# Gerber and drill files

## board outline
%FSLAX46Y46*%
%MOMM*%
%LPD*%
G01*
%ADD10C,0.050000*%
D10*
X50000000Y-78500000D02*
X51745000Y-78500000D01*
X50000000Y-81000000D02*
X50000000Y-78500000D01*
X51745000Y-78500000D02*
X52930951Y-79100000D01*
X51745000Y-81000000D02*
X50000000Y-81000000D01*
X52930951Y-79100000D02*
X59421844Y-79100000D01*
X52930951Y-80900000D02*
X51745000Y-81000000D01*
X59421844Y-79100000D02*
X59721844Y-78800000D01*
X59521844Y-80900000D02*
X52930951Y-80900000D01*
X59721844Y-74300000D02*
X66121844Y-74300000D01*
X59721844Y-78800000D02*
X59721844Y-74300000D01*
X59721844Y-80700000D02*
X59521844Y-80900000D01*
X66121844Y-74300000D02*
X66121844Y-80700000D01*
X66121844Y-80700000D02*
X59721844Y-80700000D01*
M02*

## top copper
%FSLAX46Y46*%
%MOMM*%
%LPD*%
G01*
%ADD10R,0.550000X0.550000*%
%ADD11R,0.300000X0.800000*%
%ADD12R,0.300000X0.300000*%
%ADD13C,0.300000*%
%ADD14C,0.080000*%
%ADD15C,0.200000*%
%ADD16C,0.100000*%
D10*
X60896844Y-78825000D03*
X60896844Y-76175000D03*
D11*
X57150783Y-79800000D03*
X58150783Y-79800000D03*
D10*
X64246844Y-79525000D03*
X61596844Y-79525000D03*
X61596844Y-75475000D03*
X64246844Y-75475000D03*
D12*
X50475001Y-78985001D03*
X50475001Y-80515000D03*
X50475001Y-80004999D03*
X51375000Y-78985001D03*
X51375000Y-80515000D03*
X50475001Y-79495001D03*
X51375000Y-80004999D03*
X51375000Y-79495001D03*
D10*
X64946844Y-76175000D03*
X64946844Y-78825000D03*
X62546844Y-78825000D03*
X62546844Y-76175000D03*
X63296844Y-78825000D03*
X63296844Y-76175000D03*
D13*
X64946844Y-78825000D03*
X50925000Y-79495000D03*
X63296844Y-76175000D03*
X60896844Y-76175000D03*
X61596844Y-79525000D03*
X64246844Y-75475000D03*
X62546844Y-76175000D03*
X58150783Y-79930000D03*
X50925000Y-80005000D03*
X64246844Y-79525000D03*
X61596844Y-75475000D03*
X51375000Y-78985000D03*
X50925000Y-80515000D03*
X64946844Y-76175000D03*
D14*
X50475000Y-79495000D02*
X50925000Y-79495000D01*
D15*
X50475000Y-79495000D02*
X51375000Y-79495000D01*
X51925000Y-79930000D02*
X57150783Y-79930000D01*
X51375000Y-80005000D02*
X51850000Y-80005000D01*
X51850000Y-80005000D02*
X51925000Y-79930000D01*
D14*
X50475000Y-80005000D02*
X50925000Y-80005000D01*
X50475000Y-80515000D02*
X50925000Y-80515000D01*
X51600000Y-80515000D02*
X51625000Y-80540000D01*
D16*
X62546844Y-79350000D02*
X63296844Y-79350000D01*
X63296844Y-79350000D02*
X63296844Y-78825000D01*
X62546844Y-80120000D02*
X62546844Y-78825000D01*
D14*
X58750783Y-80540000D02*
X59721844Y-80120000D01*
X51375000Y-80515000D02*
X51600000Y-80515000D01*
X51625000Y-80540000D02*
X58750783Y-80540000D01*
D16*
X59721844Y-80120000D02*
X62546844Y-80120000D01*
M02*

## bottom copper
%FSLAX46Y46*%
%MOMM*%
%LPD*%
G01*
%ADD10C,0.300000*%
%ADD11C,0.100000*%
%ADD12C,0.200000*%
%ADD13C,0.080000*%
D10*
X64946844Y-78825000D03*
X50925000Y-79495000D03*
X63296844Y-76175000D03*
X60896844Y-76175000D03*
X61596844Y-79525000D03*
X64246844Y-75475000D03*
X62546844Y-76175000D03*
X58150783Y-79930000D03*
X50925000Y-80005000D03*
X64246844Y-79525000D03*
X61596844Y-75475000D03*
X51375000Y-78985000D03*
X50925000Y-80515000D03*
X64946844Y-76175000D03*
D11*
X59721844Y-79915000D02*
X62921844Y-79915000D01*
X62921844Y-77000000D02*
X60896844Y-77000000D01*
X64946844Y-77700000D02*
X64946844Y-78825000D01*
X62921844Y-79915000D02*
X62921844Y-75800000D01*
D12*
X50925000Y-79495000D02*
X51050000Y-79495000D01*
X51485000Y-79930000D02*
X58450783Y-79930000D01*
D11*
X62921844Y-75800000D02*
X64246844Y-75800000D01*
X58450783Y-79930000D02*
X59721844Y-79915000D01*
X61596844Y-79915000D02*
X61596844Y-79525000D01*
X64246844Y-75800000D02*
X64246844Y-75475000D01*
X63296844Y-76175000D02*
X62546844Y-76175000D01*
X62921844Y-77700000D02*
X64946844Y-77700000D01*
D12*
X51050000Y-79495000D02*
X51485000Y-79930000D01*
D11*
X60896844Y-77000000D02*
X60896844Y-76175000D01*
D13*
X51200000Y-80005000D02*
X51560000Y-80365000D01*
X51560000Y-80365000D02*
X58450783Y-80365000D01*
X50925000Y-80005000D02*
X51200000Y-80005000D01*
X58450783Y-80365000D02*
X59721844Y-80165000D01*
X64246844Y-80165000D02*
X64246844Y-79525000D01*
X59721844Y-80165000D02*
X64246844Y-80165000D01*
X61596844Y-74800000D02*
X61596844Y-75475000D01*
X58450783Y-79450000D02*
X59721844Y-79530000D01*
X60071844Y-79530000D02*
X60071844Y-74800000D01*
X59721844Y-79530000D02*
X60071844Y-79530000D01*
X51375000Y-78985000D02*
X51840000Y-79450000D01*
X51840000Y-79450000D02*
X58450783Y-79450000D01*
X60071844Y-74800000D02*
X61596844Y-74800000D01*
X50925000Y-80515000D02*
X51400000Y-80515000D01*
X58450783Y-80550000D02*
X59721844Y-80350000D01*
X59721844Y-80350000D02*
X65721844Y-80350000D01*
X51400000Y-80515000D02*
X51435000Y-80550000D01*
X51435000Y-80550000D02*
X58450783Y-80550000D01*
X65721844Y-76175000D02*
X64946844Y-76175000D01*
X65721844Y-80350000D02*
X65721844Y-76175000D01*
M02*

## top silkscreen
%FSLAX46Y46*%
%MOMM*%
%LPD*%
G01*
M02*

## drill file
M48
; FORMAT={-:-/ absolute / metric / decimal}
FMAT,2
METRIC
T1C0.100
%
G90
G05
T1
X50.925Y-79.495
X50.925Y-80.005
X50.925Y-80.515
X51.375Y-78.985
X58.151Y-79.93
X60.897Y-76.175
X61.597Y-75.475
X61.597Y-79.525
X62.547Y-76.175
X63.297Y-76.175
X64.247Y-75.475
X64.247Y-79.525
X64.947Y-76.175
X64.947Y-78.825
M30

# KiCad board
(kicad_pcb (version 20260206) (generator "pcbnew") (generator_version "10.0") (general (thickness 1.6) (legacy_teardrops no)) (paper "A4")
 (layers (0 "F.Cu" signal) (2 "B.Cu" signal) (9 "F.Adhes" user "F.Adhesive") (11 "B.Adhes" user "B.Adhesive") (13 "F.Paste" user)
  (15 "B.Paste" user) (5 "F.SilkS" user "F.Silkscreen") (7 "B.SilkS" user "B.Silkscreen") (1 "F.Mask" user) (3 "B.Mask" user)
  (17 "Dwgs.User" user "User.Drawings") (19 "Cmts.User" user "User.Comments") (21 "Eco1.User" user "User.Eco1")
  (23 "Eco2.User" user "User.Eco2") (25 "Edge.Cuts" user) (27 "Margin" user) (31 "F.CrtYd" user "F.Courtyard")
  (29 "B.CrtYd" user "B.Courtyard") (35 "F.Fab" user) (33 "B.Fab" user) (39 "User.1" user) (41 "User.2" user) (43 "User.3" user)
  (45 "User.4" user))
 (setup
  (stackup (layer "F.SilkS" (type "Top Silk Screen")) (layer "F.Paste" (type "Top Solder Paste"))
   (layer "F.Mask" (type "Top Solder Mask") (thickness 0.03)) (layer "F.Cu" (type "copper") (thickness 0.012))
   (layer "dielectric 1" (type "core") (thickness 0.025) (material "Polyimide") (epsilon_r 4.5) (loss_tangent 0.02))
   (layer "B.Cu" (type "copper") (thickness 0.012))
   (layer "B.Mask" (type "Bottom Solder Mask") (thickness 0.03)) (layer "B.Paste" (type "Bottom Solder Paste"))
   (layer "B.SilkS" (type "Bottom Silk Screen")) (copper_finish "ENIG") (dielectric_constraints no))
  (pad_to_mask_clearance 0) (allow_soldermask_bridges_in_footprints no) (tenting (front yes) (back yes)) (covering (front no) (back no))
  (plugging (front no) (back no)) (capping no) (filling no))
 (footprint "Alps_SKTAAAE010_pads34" (layer "F.Cu") (at 60.521844 77.5 90)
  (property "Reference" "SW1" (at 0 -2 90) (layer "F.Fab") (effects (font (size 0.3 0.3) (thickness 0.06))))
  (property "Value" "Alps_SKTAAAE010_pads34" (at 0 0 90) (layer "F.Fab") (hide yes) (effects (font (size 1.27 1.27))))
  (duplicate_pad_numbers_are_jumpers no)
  (pad "3" smd rect (at -1.325 0.375 90) (size 0.55 0.55) (layers "F.Cu" "F.Mask") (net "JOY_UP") (solder_mask_margin 0.05)
   (thermal_bridge_angle 45))
  (pad "4" smd rect (at 1.325 0.375 90) (size 0.55 0.55) (layers "F.Cu" "F.Mask") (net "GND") (solder_mask_margin 0.05)
   (thermal_bridge_angle 45)))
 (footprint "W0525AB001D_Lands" (layer "F.Cu") (at 57.650783 79.93)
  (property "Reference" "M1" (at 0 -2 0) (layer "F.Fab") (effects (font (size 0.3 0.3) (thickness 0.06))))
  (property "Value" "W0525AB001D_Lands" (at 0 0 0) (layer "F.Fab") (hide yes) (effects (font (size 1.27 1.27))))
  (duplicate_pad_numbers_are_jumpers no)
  (pad "1" smd rect (at -0.5 -0.13) (size 0.3 0.8) (layers "F.Cu" "F.Mask") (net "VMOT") (solder_mask_margin 0.05) (thermal_bridge_angle 45))
  (pad "2" smd rect (at 0.5 -0.13) (size 0.3 0.8) (layers "F.Cu" "F.Mask") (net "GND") (solder_mask_margin 0.05) (thermal_bridge_angle 45)))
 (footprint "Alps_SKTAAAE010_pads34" (layer "F.Cu") (at 62.921844 79.9 180)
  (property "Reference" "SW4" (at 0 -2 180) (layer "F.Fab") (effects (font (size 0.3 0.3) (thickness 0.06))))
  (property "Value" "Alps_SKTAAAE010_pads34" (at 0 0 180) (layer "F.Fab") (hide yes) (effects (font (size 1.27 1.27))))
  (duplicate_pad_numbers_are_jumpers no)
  (pad "3" smd rect (at -1.325 0.375 180) (size 0.55 0.55) (layers "F.Cu" "F.Mask") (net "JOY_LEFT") (solder_mask_margin 0.05)
   (thermal_bridge_angle 45))
  (pad "4" smd rect (at 1.325 0.375 180) (size 0.55 0.55) (layers "F.Cu" "F.Mask") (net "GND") (solder_mask_margin 0.05)
   (thermal_bridge_angle 45)))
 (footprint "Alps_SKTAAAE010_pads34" (layer "F.Cu") (at 62.921844 75.1)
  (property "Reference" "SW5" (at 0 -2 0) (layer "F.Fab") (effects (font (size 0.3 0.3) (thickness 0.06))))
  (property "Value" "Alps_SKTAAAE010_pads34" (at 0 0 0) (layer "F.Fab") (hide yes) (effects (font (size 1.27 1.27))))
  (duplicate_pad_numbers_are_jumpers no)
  (pad "3" smd rect (at -1.325 0.375) (size 0.55 0.55) (layers "F.Cu" "F.Mask") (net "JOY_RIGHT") (solder_mask_margin 0.05)
   (thermal_bridge_angle 45))
  (pad "4" smd rect (at 1.325 0.375) (size 0.55 0.55) (layers "F.Cu" "F.Mask") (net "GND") (solder_mask_margin 0.05)
   (thermal_bridge_angle 45)))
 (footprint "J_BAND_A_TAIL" (layer "F.Cu") (at 50.9 79.75)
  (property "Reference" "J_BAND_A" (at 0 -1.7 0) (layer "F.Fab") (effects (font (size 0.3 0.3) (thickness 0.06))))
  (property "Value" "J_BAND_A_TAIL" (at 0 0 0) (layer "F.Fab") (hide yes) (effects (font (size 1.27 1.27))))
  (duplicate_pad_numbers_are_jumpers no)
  (pad "1" smd rect (at -0.424999 -0.764999) (size 0.3 0.3) (layers "F.Cu" "F.Mask") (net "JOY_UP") (solder_mask_margin 0.05)
   (thermal_bridge_angle 45))
  (pad "2" smd rect (at -0.424999 0.765) (size 0.3 0.3) (layers "F.Cu" "F.Mask") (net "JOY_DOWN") (solder_mask_margin 0.05)
   (thermal_bridge_angle 45))
  (pad "3" smd rect (at -0.424999 0.254999) (size 0.3 0.3) (layers "F.Cu" "F.Mask") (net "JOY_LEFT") (solder_mask_margin 0.05)
   (thermal_bridge_angle 45))
  (pad "4" smd rect (at 0.475 -0.764999) (size 0.3 0.3) (layers "F.Cu" "F.Mask") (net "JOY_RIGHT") (solder_mask_margin 0.05)
   (thermal_bridge_angle 45))
  (pad "5" smd rect (at 0.475 0.765) (size 0.3 0.3) (layers "F.Cu" "F.Mask") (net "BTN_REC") (solder_mask_margin 0.05)
   (thermal_bridge_angle 45))
  (pad "6" smd rect (at -0.424999 -0.254999) (size 0.3 0.3) (layers "F.Cu" "F.Mask") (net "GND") (solder_mask_margin 0.05)
   (thermal_bridge_angle 45))
  (pad "7" smd rect (at 0.475 0.254999) (size 0.3 0.3) (layers "F.Cu" "F.Mask") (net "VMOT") (solder_mask_margin 0.05)
   (thermal_bridge_angle 45))
  (pad "8" smd rect (at 0.475 -0.254999) (size 0.3 0.3) (layers "F.Cu" "F.Mask") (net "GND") (solder_mask_margin 0.05)
   (thermal_bridge_angle 45)))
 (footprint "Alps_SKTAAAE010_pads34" (layer "F.Cu") (at 65.321844 77.5 -90)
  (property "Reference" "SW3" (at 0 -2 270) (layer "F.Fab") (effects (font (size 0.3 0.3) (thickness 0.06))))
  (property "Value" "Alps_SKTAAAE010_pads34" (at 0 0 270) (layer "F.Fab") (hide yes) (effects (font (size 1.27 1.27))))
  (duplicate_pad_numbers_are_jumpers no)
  (pad "3" smd rect (at -1.325 0.375 270) (size 0.55 0.55) (layers "F.Cu" "F.Mask") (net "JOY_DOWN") (solder_mask_margin 0.05)
   (thermal_bridge_angle 45))
  (pad "4" smd rect (at 1.325 0.375 270) (size 0.55 0.55) (layers "F.Cu" "F.Mask") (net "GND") (solder_mask_margin 0.05)
   (thermal_bridge_angle 45)))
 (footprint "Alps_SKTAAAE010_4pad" (layer "F.Cu") (at 62.921844 77.5 90)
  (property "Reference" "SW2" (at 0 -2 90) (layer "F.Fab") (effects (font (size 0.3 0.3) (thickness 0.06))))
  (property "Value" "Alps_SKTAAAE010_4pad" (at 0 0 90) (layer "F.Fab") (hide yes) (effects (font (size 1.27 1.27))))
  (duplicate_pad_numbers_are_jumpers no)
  (pad "1" smd rect (at -1.325 -0.375 90) (size 0.55 0.55) (layers "F.Cu" "F.Mask") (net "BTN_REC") (solder_mask_margin 0.05)
   (thermal_bridge_angle 45))
  (pad "2" smd rect (at 1.325 -0.375 90) (size 0.55 0.55) (layers "F.Cu" "F.Mask") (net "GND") (solder_mask_margin 0.05)
   (thermal_bridge_angle 45))
  (pad "3" smd rect (at -1.325 0.375 90) (size 0.55 0.55) (layers "F.Cu" "F.Mask") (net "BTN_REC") (solder_mask_margin 0.05)
   (thermal_bridge_angle 45))
  (pad "4" smd rect (at 1.325 0.375 90) (size 0.55 0.55) (layers "F.Cu" "F.Mask") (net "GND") (solder_mask_margin 0.05)
   (thermal_bridge_angle 45)))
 (gr_line (start 50 78.5) (end 51.745 78.5) (stroke (width 0.05) (type default)) (layer "Edge.Cuts"))
 (gr_line (start 50 81) (end 50 78.5) (stroke (width 0.05) (type default)) (layer "Edge.Cuts"))
 (gr_line (start 51.745 78.5) (end 52.930951 79.1) (stroke (width 0.05) (type default)) (layer "Edge.Cuts"))
 (gr_line (start 51.745 81) (end 50 81) (stroke (width 0.05) (type default)) (layer "Edge.Cuts"))
 (gr_line (start 52.930951 79.1) (end 59.421844 79.1) (stroke (width 0.05) (type default)) (layer "Edge.Cuts"))
 (gr_line (start 52.930951 80.9) (end 51.745 81) (stroke (width 0.05) (type default)) (layer "Edge.Cuts"))
 (gr_line (start 59.421844 79.1) (end 59.721844 78.8) (stroke (width 0.05) (type default)) (layer "Edge.Cuts"))
 (gr_line (start 59.521844 80.9) (end 52.930951 80.9) (stroke (width 0.05) (type default)) (layer "Edge.Cuts"))
 (gr_line (start 59.721844 74.3) (end 66.121844 74.3) (stroke (width 0.05) (type default)) (layer "Edge.Cuts"))
 (gr_line (start 59.721844 78.8) (end 59.721844 74.3) (stroke (width 0.05) (type default)) (layer "Edge.Cuts"))
 (gr_line (start 59.721844 80.7) (end 59.521844 80.9) (stroke (width 0.05) (type default)) (layer "Edge.Cuts"))
 (gr_line (start 66.121844 74.3) (end 66.121844 80.7) (stroke (width 0.05) (type default)) (layer "Edge.Cuts"))
 (gr_line (start 66.121844 80.7) (end 59.721844 80.7) (stroke (width 0.05) (type default)) (layer "Edge.Cuts"))
 (segment (start 50.475 79.495) (end 50.925 79.495) (width 0.08) (layer "F.Cu") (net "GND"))
 (segment (start 50.475 79.495) (end 51.375 79.495) (width 0.2) (layer "F.Cu") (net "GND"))
 (via (at 64.946844 78.825) (size 0.3) (drill 0.1) (layers "F.Cu" "B.Cu") (tenting (front yes) (back yes)) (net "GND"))
 (via (at 50.925 79.495) (size 0.3) (drill 0.1) (layers "F.Cu" "B.Cu") (tenting (front yes) (back yes)) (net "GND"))
 (via (at 63.296844 76.175) (size 0.3) (drill 0.1) (layers "F.Cu" "B.Cu") (tenting (front yes) (back yes)) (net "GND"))
 (via (at 60.896844 76.175) (size 0.3) (drill 0.1) (layers "F.Cu" "B.Cu") (tenting (front yes) (back yes)) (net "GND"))
 (via (at 61.596844 79.525) (size 0.3) (drill 0.1) (layers "F.Cu" "B.Cu") (tenting (front yes) (back yes)) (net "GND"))
 (via (at 64.246844 75.475) (size 0.3) (drill 0.1) (layers "F.Cu" "B.Cu") (tenting (front yes) (back yes)) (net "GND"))
 (via (at 62.546844 76.175) (size 0.3) (drill 0.1) (layers "F.Cu" "B.Cu") (tenting (front yes) (back yes)) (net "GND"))
 (via (at 58.150783 79.93) (size 0.3) (drill 0.1) (layers "F.Cu" "B.Cu") (tenting (front yes) (back yes)) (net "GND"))
 (segment (start 59.721844 79.915) (end 62.921844 79.915) (width 0.1) (layer "B.Cu") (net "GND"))
 (segment (start 62.921844 77) (end 60.896844 77) (width 0.1) (layer "B.Cu") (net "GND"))
 (segment (start 64.946844 77.7) (end 64.946844 78.825) (width 0.1) (layer "B.Cu") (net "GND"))
 (segment (start 62.921844 79.915) (end 62.921844 75.8) (width 0.1) (layer "B.Cu") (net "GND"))
 (segment (start 50.925 79.495) (end 51.05 79.495) (width 0.2) (layer "B.Cu") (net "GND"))
 (segment (start 51.485 79.93) (end 58.450783 79.93) (width 0.2) (layer "B.Cu") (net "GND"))
 (segment (start 62.921844 75.8) (end 64.246844 75.8) (width 0.1) (layer "B.Cu") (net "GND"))
 (segment (start 58.450783 79.93) (end 59.721844 79.915) (width 0.1) (layer "B.Cu") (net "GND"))
 (segment (start 61.596844 79.915) (end 61.596844 79.525) (width 0.1) (layer "B.Cu") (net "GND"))
 (segment (start 64.246844 75.8) (end 64.246844 75.475) (width 0.1) (layer "B.Cu") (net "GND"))
 (segment (start 63.296844 76.175) (end 62.546844 76.175) (width 0.1) (layer "B.Cu") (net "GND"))
 (segment (start 62.921844 77.7) (end 64.946844 77.7) (width 0.1) (layer "B.Cu") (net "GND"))
 (segment (start 51.05 79.495) (end 51.485 79.93) (width 0.2) (layer "B.Cu") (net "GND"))
 (segment (start 60.896844 77) (end 60.896844 76.175) (width 0.1) (layer "B.Cu") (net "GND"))
 (segment (start 51.925 79.93) (end 57.150783 79.93) (width 0.2) (layer "F.Cu") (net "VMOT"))
 (segment (start 51.375 80.005) (end 51.85 80.005) (width 0.2) (layer "F.Cu") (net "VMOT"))
 (segment (start 51.85 80.005) (end 51.925 79.93) (width 0.2) (layer "F.Cu") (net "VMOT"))
 (segment (start 50.475 80.005) (end 50.925 80.005) (width 0.08) (layer "F.Cu") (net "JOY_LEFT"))
 (via (at 50.925 80.005) (size 0.3) (drill 0.1) (layers "F.Cu" "B.Cu") (tenting (front yes) (back yes)) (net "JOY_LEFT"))
 (via (at 64.246844 79.525) (size 0.3) (drill 0.1) (layers "F.Cu" "B.Cu") (tenting (front yes) (back yes)) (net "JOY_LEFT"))
 (segment (start 51.2 80.005) (end 51.56 80.365) (width 0.08) (layer "B.Cu") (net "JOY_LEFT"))
 (segment (start 51.56 80.365) (end 58.450783 80.365) (width 0.08) (layer "B.Cu") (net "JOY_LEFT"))
 (segment (start 50.925 80.005) (end 51.2 80.005) (width 0.08) (layer "B.Cu") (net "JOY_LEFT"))
 (segment (start 58.450783 80.365) (end 59.721844 80.165) (width 0.08) (layer "B.Cu") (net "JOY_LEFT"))
 (segment (start 64.246844 80.165) (end 64.246844 79.525) (width 0.08) (layer "B.Cu") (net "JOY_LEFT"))
 (segment (start 59.721844 80.165) (end 64.246844 80.165) (width 0.08) (layer "B.Cu") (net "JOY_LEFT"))
 (via (at 61.596844 75.475) (size 0.3) (drill 0.1) (layers "F.Cu" "B.Cu") (tenting (front yes) (back yes)) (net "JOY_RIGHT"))
 (via (at 51.375 78.985) (size 0.3) (drill 0.1) (layers "F.Cu" "B.Cu") (tenting (front yes) (back yes)) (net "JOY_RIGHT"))
 (segment (start 61.596844 74.8) (end 61.596844 75.475) (width 0.08) (layer "B.Cu") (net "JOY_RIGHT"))
 (segment (start 58.450783 79.45) (end 59.721844 79.53) (width 0.08) (layer "B.Cu") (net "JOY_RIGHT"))
 (segment (start 60.071844 79.53) (end 60.071844 74.8) (width 0.08) (layer "B.Cu") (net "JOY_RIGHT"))
 (segment (start 59.721844 79.53) (end 60.071844 79.53) (width 0.08) (layer "B.Cu") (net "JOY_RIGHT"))
 (segment (start 51.375 78.985) (end 51.84 79.45) (width 0.08) (layer "B.Cu") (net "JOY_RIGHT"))
 (segment (start 51.84 79.45) (end 58.450783 79.45) (width 0.08) (layer "B.Cu") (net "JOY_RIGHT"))
 (segment (start 60.071844 74.8) (end 61.596844 74.8) (width 0.08) (layer "B.Cu") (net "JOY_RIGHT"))
 (segment (start 50.475 80.515) (end 50.925 80.515) (width 0.08) (layer "F.Cu") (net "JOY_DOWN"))
 (via (at 50.925 80.515) (size 0.3) (drill 0.1) (layers "F.Cu" "B.Cu") (tenting (front yes) (back yes)) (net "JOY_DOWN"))
 (via (at 64.946844 76.175) (size 0.3) (drill 0.1) (layers "F.Cu" "B.Cu") (tenting (front yes) (back yes)) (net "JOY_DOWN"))
 (segment (start 50.925 80.515) (end 51.4 80.515) (width 0.08) (layer "B.Cu") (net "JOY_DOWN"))
 (segment (start 58.450783 80.55) (end 59.721844 80.35) (width 0.08) (layer "B.Cu") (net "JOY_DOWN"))
 (segment (start 59.721844 80.35) (end 65.721844 80.35) (width 0.08) (layer "B.Cu") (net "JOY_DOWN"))
 (segment (start 51.4 80.515) (end 51.435 80.55) (width 0.08) (layer "B.Cu") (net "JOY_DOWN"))
 (segment (start 51.435 80.55) (end 58.450783 80.55) (width 0.08) (layer "B.Cu") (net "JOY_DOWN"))
 (segment (start 65.721844 76.175) (end 64.946844 76.175) (width 0.08) (layer "B.Cu") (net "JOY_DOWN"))
 (segment (start 65.721844 80.35) (end 65.721844 76.175) (width 0.08) (layer "B.Cu") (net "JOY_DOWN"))
 (segment (start 51.6 80.515) (end 51.625 80.54) (width 0.08) (layer "F.Cu") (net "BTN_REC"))
 (segment (start 62.546844 79.35) (end 63.296844 79.35) (width 0.1) (layer "F.Cu") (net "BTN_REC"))
 (segment (start 63.296844 79.35) (end 63.296844 78.825) (width 0.1) (layer "F.Cu") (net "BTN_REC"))
 (segment (start 62.546844 80.12) (end 62.546844 78.825) (width 0.1) (layer "F.Cu") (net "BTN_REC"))
 (segment (start 58.750783 80.54) (end 59.721844 80.12) (width 0.08) (layer "F.Cu") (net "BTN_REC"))
 (segment (start 51.375 80.515) (end 51.6 80.515) (width 0.08) (layer "F.Cu") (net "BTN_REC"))
 (segment (start 51.625 80.54) (end 58.750783 80.54) (width 0.08) (layer "F.Cu") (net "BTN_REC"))
 (segment (start 59.721844 80.12) (end 62.546844 80.12) (width 0.1) (layer "F.Cu") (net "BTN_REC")))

